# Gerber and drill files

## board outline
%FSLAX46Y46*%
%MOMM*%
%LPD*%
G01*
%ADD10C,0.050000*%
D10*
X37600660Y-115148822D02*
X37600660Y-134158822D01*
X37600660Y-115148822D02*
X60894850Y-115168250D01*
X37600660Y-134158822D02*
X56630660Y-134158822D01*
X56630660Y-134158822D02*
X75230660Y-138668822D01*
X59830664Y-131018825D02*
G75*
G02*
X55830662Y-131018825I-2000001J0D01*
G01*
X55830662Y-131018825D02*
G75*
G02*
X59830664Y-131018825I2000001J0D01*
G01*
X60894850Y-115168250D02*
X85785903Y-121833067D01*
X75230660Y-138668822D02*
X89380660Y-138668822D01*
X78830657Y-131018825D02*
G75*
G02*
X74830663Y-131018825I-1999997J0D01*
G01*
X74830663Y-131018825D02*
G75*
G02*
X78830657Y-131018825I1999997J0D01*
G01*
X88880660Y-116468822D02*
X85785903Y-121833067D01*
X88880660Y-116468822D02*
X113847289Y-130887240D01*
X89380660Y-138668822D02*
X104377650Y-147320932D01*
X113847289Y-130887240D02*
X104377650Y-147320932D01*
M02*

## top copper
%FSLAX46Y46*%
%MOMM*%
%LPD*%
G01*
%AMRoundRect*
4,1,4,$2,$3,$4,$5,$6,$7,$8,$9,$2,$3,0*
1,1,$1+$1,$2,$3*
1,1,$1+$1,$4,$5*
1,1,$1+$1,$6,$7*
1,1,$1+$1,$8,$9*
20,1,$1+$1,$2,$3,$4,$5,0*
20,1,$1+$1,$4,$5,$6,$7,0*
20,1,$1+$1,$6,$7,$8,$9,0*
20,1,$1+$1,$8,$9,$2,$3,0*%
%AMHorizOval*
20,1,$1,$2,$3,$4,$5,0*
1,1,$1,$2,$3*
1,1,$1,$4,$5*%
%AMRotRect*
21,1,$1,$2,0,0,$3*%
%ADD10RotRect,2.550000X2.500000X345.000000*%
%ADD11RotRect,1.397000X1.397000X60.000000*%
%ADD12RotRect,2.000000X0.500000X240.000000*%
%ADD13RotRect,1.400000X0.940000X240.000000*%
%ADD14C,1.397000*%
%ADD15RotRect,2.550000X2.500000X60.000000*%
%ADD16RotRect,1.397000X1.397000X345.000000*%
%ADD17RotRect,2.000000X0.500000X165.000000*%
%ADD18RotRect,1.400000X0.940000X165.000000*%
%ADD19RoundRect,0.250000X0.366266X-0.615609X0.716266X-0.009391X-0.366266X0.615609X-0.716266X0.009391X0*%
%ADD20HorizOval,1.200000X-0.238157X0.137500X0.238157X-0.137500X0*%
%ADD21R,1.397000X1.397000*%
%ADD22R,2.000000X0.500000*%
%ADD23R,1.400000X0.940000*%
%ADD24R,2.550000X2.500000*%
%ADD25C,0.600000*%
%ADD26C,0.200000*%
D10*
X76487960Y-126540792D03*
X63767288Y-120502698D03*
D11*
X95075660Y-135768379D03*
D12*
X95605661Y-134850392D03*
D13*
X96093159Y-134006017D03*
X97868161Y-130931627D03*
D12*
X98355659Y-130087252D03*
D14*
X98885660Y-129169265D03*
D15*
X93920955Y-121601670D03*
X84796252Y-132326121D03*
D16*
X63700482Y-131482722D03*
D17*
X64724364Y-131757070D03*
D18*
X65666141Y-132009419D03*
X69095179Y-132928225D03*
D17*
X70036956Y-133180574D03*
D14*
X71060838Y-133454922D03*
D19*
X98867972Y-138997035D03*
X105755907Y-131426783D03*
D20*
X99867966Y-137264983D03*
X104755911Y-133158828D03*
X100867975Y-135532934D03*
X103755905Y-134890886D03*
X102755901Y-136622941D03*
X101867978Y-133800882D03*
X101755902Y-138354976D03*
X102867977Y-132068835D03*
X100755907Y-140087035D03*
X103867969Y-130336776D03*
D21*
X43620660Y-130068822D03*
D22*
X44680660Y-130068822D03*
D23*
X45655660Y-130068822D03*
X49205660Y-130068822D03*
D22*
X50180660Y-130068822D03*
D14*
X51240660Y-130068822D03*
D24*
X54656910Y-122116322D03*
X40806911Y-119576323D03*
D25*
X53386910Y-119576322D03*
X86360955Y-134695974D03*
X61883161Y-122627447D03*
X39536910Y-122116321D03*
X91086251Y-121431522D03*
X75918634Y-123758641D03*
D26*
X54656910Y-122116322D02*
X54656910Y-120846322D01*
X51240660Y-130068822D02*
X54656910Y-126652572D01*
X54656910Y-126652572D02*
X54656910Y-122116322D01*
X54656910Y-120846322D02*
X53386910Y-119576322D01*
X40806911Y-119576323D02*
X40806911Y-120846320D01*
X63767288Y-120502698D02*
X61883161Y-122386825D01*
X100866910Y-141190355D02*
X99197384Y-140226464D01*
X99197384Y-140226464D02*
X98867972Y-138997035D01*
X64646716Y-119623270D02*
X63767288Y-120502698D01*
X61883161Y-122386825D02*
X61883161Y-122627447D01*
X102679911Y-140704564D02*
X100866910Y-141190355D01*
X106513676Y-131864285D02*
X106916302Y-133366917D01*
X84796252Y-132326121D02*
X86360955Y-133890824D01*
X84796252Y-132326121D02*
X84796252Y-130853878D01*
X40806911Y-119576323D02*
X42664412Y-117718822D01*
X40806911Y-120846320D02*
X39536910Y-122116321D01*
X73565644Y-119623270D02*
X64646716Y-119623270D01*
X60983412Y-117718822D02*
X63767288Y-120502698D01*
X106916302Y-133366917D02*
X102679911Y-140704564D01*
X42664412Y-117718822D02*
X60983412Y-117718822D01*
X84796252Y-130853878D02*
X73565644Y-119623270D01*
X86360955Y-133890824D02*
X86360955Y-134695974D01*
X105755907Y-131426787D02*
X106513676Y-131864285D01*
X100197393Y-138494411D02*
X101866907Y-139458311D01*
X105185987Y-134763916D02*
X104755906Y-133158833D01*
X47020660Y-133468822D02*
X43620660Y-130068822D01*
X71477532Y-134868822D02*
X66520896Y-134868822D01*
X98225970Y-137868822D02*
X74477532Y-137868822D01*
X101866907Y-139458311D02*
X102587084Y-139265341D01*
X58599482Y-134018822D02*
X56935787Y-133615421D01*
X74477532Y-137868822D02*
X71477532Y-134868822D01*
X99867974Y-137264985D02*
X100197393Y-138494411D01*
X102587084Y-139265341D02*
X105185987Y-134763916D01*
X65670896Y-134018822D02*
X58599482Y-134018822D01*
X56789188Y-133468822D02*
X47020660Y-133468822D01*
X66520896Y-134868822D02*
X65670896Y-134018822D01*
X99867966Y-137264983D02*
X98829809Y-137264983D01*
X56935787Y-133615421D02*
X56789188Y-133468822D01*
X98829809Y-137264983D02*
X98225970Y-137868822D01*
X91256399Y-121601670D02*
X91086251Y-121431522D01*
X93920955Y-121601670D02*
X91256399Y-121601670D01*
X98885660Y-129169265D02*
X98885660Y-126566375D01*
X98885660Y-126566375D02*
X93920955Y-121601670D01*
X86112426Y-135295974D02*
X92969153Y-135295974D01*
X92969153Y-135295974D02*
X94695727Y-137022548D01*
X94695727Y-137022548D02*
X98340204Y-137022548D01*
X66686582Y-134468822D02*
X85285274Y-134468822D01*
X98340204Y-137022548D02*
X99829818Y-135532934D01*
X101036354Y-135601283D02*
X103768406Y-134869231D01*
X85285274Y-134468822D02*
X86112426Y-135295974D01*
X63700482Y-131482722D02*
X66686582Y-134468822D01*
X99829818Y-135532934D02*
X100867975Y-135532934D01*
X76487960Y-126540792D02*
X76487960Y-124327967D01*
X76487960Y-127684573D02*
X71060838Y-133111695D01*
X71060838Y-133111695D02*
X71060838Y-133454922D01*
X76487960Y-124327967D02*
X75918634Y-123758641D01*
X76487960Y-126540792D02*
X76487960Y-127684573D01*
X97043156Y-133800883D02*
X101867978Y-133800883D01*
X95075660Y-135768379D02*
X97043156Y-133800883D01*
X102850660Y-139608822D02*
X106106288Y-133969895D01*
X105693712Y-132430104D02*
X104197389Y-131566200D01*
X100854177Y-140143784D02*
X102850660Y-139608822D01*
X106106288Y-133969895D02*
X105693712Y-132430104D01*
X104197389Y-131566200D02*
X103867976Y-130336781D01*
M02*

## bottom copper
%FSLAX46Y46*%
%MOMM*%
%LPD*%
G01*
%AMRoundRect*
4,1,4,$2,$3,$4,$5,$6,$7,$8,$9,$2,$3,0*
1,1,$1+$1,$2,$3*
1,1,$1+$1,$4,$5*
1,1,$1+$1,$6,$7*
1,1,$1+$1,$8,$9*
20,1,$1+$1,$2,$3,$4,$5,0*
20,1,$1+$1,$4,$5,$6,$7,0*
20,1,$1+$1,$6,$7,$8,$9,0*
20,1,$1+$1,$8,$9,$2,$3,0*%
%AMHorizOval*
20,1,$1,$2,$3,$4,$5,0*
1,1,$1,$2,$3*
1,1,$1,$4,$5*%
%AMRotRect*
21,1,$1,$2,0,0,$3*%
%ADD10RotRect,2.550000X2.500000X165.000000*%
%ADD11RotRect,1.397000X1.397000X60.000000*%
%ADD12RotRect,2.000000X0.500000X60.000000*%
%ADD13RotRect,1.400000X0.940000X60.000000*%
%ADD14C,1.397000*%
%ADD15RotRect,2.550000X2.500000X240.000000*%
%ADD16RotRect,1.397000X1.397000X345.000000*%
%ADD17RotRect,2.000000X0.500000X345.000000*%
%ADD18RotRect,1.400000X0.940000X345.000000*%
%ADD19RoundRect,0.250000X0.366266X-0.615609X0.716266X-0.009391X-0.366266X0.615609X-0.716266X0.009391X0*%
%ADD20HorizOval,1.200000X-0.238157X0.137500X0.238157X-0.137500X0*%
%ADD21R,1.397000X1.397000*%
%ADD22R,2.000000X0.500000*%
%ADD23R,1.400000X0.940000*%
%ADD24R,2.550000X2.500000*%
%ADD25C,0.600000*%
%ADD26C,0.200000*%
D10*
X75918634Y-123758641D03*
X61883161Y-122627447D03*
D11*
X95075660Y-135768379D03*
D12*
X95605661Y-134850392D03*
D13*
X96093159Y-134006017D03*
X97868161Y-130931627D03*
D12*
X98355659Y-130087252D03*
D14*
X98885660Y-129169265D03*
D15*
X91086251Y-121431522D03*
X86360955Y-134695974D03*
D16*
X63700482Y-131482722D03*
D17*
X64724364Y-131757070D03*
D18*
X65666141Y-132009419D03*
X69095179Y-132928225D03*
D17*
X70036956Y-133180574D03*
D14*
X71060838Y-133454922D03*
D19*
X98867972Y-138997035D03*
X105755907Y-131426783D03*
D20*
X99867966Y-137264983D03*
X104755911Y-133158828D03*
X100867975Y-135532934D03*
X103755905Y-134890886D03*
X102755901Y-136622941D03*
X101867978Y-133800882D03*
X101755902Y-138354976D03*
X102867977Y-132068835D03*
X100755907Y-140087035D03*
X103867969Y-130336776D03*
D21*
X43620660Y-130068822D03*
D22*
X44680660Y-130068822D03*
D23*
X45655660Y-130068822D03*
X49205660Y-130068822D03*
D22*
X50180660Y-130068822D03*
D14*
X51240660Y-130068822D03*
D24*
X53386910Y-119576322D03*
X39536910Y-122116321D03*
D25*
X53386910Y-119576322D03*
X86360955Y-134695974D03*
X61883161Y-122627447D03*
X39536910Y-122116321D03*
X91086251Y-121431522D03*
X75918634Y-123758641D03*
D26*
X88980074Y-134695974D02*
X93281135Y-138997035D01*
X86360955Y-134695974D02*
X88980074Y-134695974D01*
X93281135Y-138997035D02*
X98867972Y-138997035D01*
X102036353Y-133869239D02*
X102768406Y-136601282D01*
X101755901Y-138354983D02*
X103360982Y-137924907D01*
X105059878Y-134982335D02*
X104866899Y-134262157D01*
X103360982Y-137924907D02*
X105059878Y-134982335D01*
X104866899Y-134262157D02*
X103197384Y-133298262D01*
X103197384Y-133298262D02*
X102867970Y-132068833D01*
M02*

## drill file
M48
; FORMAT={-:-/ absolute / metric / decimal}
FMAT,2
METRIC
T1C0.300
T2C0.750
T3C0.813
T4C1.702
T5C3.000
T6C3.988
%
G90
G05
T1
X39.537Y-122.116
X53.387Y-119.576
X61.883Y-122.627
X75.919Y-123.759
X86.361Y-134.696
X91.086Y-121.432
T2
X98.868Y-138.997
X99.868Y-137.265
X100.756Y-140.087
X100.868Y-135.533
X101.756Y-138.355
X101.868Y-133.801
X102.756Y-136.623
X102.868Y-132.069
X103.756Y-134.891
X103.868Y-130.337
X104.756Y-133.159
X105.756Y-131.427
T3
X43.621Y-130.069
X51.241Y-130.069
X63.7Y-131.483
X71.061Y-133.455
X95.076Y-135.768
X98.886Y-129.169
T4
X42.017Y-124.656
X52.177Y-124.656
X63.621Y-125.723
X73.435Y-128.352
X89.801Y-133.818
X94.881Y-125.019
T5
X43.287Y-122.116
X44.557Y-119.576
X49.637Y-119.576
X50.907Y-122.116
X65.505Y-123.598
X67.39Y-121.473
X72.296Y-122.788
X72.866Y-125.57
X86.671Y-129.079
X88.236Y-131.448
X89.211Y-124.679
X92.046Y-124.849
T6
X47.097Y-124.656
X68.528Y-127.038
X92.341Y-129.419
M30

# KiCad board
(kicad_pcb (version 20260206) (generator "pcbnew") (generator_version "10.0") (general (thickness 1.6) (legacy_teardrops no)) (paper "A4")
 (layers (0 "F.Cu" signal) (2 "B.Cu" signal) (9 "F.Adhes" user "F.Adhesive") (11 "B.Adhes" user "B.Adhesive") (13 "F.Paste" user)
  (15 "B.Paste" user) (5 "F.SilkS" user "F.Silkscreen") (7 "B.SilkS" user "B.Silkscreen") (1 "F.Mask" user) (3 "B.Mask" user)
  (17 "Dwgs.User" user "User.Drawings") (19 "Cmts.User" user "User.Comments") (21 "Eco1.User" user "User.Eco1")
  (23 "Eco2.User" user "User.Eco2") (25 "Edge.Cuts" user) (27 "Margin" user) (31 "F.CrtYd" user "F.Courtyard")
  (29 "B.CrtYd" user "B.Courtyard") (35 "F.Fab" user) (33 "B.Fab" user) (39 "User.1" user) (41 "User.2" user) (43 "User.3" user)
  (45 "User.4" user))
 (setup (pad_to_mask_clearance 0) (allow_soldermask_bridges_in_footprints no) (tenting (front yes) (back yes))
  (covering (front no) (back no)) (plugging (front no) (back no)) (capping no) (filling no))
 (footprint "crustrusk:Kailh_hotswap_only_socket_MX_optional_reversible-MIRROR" (layer "F.Cu") (at 68.52816 127.037572 -15)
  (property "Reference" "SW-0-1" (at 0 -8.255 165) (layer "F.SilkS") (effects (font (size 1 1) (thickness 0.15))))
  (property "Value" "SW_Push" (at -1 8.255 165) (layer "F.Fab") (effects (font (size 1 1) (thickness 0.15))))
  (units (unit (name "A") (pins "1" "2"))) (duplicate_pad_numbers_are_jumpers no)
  (pad "" np_thru_hole circle (at -5.08 0 345) (size 1.7018 1.7018) (drill 1.7018) (layers "*.Cu" "*.Mask"))
  (pad "" np_thru_hole circle (at -3.81 -2.54 165) (size 3 3) (drill 3) (layers "*.Cu" "*.Mask"))
  (pad "" np_thru_hole circle (at -2.54 -5.079998 345) (size 3 3) (drill 3) (layers "*.Cu" "*.Mask"))
  (pad "" np_thru_hole circle (at 0 0 345) (size 3.9878 3.9878) (drill 3.9878) (layers "*.Cu" "*.Mask"))
  (pad "" np_thru_hole circle (at 2.540003 -5.080001 165) (size 3 3) (drill 3) (layers "*.Cu" "*.Mask"))
  (pad "" np_thru_hole circle (at 3.81 -2.54 345) (size 3 3) (drill 3) (layers "*.Cu" "*.Mask"))
  (pad "" np_thru_hole circle (at 5.08 0 345) (size 1.7018 1.7018) (drill 1.7018) (layers "*.Cu" "*.Mask"))
  (pad "1" smd rect (at 6.29 -5.08 165) (size 2.55 2.5) (layers "B.Cu" "B.Mask" "B.Paste") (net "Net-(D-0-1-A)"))
  (pad "1" smd rect (at 7.56 -2.54 345) (size 2.55 2.5) (layers "F.Cu" "F.Mask" "F.Paste") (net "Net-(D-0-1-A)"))
  (pad "2" smd rect (at -7.56 -2.540001 165) (size 2.55 2.5) (layers "B.Cu" "B.Mask" "B.Paste") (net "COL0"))
  (pad "2" smd rect (at -6.289999 -5.079999 345) (size 2.55 2.5) (layers "F.Cu" "F.Mask" "F.Paste") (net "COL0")))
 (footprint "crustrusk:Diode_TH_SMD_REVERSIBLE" (layer "F.Cu") (at 96.98066 132.468822 60)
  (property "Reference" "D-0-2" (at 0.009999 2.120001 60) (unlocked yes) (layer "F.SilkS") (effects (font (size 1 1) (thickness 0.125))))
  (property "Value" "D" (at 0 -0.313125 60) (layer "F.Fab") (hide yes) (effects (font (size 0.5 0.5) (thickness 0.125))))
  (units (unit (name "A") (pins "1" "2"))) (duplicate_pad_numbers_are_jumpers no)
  (pad "1" thru_hole rect (at -3.81 0 60) (size 1.397 1.397) (drill 0.8128) (layers "*.Cu" "*.Mask") (remove_unused_layers no)
   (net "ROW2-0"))
  (pad "1" smd rect (at -2.75 0.000001 240) (size 2 0.5) (layers "F.Cu") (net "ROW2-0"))
  (pad "1" smd rect (at -2.75 0.000001 60) (size 2 0.5) (layers "B.Cu") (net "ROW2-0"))
  (pad "1" smd rect (at -1.775 -0.000001 240) (size 1.4 0.94) (layers "F.Cu" "F.Mask" "F.Paste") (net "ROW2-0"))
  (pad "1" smd rect (at -1.775 -0.000001 60) (size 1.4 0.94) (layers "B.Cu" "B.Mask" "B.Paste") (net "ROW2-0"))
  (pad "2" smd rect (at 1.775 0.000001 240) (size 1.4 0.94) (layers "F.Cu" "F.Mask" "F.Paste") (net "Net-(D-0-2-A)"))
  (pad "2" smd rect (at 1.775 0.000001 60) (size 1.4 0.94) (layers "B.Cu" "B.Mask" "B.Paste") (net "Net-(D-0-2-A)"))
  (pad "2" smd rect (at 2.75 -0.000001 240) (size 2 0.5) (layers "F.Cu") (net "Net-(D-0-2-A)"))
  (pad "2" smd rect (at 2.75 -0.000001 60) (size 2 0.5) (layers "B.Cu") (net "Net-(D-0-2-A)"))
  (pad "2" thru_hole circle (at 3.81 0 60) (size 1.397 1.397) (drill 0.8128) (layers "*.Cu" "*.Mask") (remove_unused_layers no)
   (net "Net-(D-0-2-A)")))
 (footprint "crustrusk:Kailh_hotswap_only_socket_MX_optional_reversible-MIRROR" (layer "F.Cu") (at 92.34066 129.418822 60)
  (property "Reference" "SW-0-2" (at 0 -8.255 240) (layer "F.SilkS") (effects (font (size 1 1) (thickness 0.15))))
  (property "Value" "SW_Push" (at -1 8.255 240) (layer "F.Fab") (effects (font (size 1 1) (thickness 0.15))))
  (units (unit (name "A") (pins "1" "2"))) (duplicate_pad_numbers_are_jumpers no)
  (pad "" np_thru_hole circle (at -5.08 0 60) (size 1.7018 1.7018) (drill 1.7018) (layers "*.Cu" "*.Mask"))
  (pad "" np_thru_hole circle (at -3.81 -2.54 240) (size 3 3) (drill 3) (layers "*.Cu" "*.Mask"))
  (pad "" np_thru_hole circle (at -2.54 -5.079997 60) (size 3 3) (drill 3) (layers "*.Cu" "*.Mask"))
  (pad "" np_thru_hole circle (at 0 0 60) (size 3.9878 3.9878) (drill 3.9878) (layers "*.Cu" "*.Mask"))
  (pad "" np_thru_hole circle (at 2.540002 -5.080001 240) (size 3 3) (drill 3) (layers "*.Cu" "*.Mask"))
  (pad "" np_thru_hole circle (at 3.81 -2.540001 60) (size 3 3) (drill 3) (layers "*.Cu" "*.Mask"))
  (pad "" np_thru_hole circle (at 5.08 0 60) (size 1.7018 1.7018) (drill 1.7018) (layers "*.Cu" "*.Mask"))
  (pad "1" smd rect (at 6.29 -5.08 240) (size 2.55 2.5) (layers "B.Cu" "B.Mask" "B.Paste") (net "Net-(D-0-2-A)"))
  (pad "1" smd rect (at 7.56 -2.54 60) (size 2.55 2.5) (layers "F.Cu" "F.Mask" "F.Paste") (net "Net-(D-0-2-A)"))
  (pad "2" smd rect (at -7.56 -2.54 240) (size 2.55 2.5) (layers "B.Cu" "B.Mask" "B.Paste") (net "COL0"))
  (pad "2" smd rect (at -6.289999 -5.079999 60) (size 2.55 2.5) (layers "F.Cu" "F.Mask" "F.Paste") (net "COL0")))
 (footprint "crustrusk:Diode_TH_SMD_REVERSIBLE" (layer "F.Cu") (at 67.38066 132.468822 -15)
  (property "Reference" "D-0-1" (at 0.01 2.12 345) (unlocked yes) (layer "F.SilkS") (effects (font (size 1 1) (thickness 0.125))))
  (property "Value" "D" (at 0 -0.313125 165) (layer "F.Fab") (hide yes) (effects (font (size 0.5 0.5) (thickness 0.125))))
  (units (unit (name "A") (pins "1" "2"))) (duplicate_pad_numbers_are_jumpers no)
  (pad "1" thru_hole rect (at -3.81 0.000001 345) (size 1.397 1.397) (drill 0.8128) (layers "*.Cu" "*.Mask") (remove_unused_layers no)
   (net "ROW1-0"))
  (pad "1" smd rect (at -2.75 0 165) (size 2 0.5) (layers "F.Cu") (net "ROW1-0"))
  (pad "1" smd rect (at -2.75 0 345) (size 2 0.5) (layers "B.Cu") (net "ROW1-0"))
  (pad "1" smd rect (at -1.775 0.000001 165) (size 1.4 0.94) (layers "F.Cu" "F.Mask" "F.Paste") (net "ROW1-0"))
  (pad "1" smd rect (at -1.775 0.000001 345) (size 1.4 0.94) (layers "B.Cu" "B.Mask" "B.Paste") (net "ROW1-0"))
  (pad "2" smd rect (at 1.775 -0.000001 165) (size 1.4 0.94) (layers "F.Cu" "F.Mask" "F.Paste") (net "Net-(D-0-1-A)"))
  (pad "2" smd rect (at 1.775 -0.000001 345) (size 1.4 0.94) (layers "B.Cu" "B.Mask" "B.Paste") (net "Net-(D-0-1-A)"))
  (pad "2" smd rect (at 2.75 0 165) (size 2 0.5) (layers "F.Cu") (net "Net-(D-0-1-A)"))
  (pad "2" smd rect (at 2.75 0 345) (size 2 0.5) (layers "B.Cu") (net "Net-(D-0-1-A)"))
  (pad "2" thru_hole circle (at 3.81 -0.000001 345) (size 1.397 1.397) (drill 0.8128) (layers "*.Cu" "*.Mask") (remove_unused_layers no)
   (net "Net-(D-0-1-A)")))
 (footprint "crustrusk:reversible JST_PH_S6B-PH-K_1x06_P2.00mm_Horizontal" (layer "F.Cu") (at 98.867972 138.997035 60)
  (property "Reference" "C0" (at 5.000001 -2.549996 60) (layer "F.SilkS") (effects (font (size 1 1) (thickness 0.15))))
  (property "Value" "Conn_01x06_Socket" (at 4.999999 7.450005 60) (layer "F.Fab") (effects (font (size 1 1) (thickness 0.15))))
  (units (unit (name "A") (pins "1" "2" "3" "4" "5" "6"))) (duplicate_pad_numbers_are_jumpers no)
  (pad "1" thru_hole roundrect (at 0 0 60) (size 1.2 1.75) (drill 0.75) (layers "*.Cu" "*.Mask") (remove_unused_layers no)
   (roundrect_rratio 0.208333) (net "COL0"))
  (pad "1" thru_hole roundrect (at 9.999998 2.180001 60) (size 1.2 1.75) (drill 0.75) (layers "*.Cu" "*.Mask") (remove_unused_layers no)
   (roundrect_rratio 0.208333) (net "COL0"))
  (pad "2" thru_hole oval (at 1.999998 -0.000006 60) (size 1.2 1.75) (drill 0.75) (layers "*.Cu" "*.Mask") (remove_unused_layers no)
   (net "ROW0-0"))
  (pad "2" thru_hole oval (at 8.000005 2.180001 60) (size 1.2 1.75) (drill 0.75) (layers "*.Cu" "*.Mask") (remove_unused_layers no)
   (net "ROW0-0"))
  (pad "3" thru_hole oval (at 4.000001 0.000003 60) (size 1.2 1.75) (drill 0.75) (layers "*.Cu" "*.Mask") (remove_unused_layers no)
   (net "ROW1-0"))
  (pad "3" thru_hole oval (at 5.999996 2.18 60) (size 1.2 1.75) (drill 0.75) (layers "*.Cu" "*.Mask") (remove_unused_layers no)
   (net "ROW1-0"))
  (pad "4" thru_hole oval (at 3.99999 2.179998 60) (size 1.2 1.75) (drill 0.75) (layers "*.Cu" "*.Mask") (remove_unused_layers no)
   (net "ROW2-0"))
  (pad "4" thru_hole oval (at 6.000003 0.000005 60) (size 1.2 1.75) (drill 0.75) (layers "*.Cu" "*.Mask") (remove_unused_layers no)
   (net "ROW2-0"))
  (pad "5" thru_hole oval (at 2.000004 2.179991 60) (size 1.2 1.75) (drill 0.75) (layers "*.Cu" "*.Mask") (remove_unused_layers no)
   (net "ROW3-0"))
  (pad "5" thru_hole oval (at 8 0.000006 60) (size 1.2 1.75) (drill 0.75) (layers "*.Cu" "*.Mask") (remove_unused_layers no) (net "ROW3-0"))
  (pad "6" thru_hole oval (at 0 2.18 60) (size 1.2 1.75) (drill 0.75) (layers "*.Cu" "*.Mask") (remove_unused_layers no) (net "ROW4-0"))
  (pad "6" thru_hole oval (at 10.000003 -0.000005 60) (size 1.2 1.75) (drill 0.75) (layers "*.Cu" "*.Mask") (remove_unused_layers no)
   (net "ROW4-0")))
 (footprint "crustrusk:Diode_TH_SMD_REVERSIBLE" (layer "F.Cu") (at 47.43066 130.068822)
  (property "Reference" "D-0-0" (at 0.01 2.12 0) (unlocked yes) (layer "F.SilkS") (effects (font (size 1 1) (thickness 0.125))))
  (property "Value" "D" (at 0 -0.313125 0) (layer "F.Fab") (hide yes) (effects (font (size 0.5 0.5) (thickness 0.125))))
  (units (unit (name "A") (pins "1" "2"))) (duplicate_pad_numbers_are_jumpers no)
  (pad "1" thru_hole rect (at -3.81 0) (size 1.397 1.397) (drill 0.8128) (layers "*.Cu" "*.Mask") (remove_unused_layers no) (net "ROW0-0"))
  (pad "1" smd rect (at -2.75 0 180) (size 2 0.5) (layers "F.Cu") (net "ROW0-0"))
  (pad "1" smd rect (at -2.75 0) (size 2 0.5) (layers "B.Cu") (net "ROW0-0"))
  (pad "1" smd rect (at -1.775 0 180) (size 1.4 0.94) (layers "F.Cu" "F.Mask" "F.Paste") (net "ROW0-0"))
  (pad "1" smd rect (at -1.775 0) (size 1.4 0.94) (layers "B.Cu" "B.Mask" "B.Paste") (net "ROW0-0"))
  (pad "2" smd rect (at 1.775 0 180) (size 1.4 0.94) (layers "F.Cu" "F.Mask" "F.Paste") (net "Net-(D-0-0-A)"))
  (pad "2" smd rect (at 1.775 0) (size 1.4 0.94) (layers "B.Cu" "B.Mask" "B.Paste") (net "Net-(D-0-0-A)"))
  (pad "2" smd rect (at 2.75 0 180) (size 2 0.5) (layers "F.Cu") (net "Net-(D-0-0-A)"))
  (pad "2" smd rect (at 2.75 0) (size 2 0.5) (layers "B.Cu") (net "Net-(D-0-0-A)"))
  (pad "2" thru_hole circle (at 3.81 0) (size 1.397 1.397) (drill 0.8128) (layers "*.Cu" "*.Mask") (remove_unused_layers no)
   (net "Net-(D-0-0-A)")))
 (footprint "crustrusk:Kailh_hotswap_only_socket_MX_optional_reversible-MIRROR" (layer "F.Cu") (at 47.09691 124.656322)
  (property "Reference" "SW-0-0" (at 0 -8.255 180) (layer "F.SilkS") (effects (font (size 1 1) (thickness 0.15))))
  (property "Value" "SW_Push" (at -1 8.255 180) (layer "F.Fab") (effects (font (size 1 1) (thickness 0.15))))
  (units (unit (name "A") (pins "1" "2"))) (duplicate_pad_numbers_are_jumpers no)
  (pad "" np_thru_hole circle (at -5.08 0) (size 1.7018 1.7018) (drill 1.7018) (layers "*.Cu" "*.Mask"))
  (pad "" np_thru_hole circle (at -3.81 -2.54 180) (size 3 3) (drill 3) (layers "*.Cu" "*.Mask"))
  (pad "" np_thru_hole circle (at -2.54 -5.079998) (size 3 3) (drill 3) (layers "*.Cu" "*.Mask"))
  (pad "" np_thru_hole circle (at 0 0) (size 3.9878 3.9878) (drill 3.9878) (layers "*.Cu" "*.Mask"))
  (pad "" np_thru_hole circle (at 2.540002 -5.080001 180) (size 3 3) (drill 3) (layers "*.Cu" "*.Mask"))
  (pad "" np_thru_hole circle (at 3.81 -2.54) (size 3 3) (drill 3) (layers "*.Cu" "*.Mask"))
  (pad "" np_thru_hole circle (at 5.08 0) (size 1.7018 1.7018) (drill 1.7018) (layers "*.Cu" "*.Mask"))
  (pad "1" smd rect (at 6.29 -5.08 180) (size 2.55 2.5) (layers "B.Cu" "B.Mask" "B.Paste") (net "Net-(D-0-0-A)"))
  (pad "1" smd rect (at 7.56 -2.54) (size 2.55 2.5) (layers "F.Cu" "F.Mask" "F.Paste") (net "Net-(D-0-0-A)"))
  (pad "2" smd rect (at -7.56 -2.540001 180) (size 2.55 2.5) (layers "B.Cu" "B.Mask" "B.Paste") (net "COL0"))
  (pad "2" smd rect (at -6.289999 -5.079999) (size 2.55 2.5) (layers "F.Cu" "F.Mask" "F.Paste") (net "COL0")))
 (gr_line (start 37.60066 115.148822) (end 37.60066 134.158822) (stroke (width 0.05) (type default)) (layer "Edge.Cuts"))
 (gr_line (start 37.60066 115.148822) (end 60.89485 115.16825) (stroke (width 0.05) (type default)) (layer "Edge.Cuts"))
 (gr_line (start 37.60066 134.158822) (end 56.63066 134.158822) (stroke (width 0.05) (type default)) (layer "Edge.Cuts"))
 (gr_line (start 56.63066 134.158822) (end 75.23066 138.668822) (stroke (width 0.05) (type default)) (layer "Edge.Cuts"))
 (gr_circle (center 57.830663 131.018825) (end 55.830662 131.018825) (stroke (width 0.05) (type default)) (fill no) (layer "Edge.Cuts"))
 (gr_line (start 60.89485 115.16825) (end 85.785903 121.833067) (stroke (width 0.05) (type default)) (layer "Edge.Cuts"))
 (gr_line (start 75.23066 138.668822) (end 89.38066 138.668822) (stroke (width 0.05) (type default)) (layer "Edge.Cuts"))
 (gr_circle (center 76.83066 131.018825) (end 74.830663 131.018825) (stroke (width 0.05) (type default)) (fill no) (layer "Edge.Cuts"))
 (gr_line (start 88.88066 116.468822) (end 85.785903 121.833067) (stroke (width 0.05) (type default)) (layer "Edge.Cuts"))
 (gr_line (start 88.88066 116.468822) (end 113.847289 130.88724) (stroke (width 0.05) (type default)) (layer "Edge.Cuts"))
 (gr_line (start 89.38066 138.668822) (end 104.37765 147.320932) (stroke (width 0.05) (type default)) (layer "Edge.Cuts"))
 (gr_line (start 113.847289 130.88724) (end 104.37765 147.320932) (stroke (width 0.05) (type default)) (layer "Edge.Cuts"))
 (segment (start 54.65691 122.116322) (end 54.65691 120.846322) (width 0.2) (layer "F.Cu") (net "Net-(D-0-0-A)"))
 (segment (start 51.24066 130.068822) (end 54.65691 126.652572) (width 0.2) (layer "F.Cu") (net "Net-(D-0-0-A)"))
 (segment (start 54.65691 126.652572) (end 54.65691 122.116322) (width 0.2) (layer "F.Cu") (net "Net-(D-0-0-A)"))
 (segment (start 54.65691 120.846322) (end 53.38691 119.576322) (width 0.2) (layer "F.Cu") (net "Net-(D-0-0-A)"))
 (via (at 53.38691 119.576322) (size 0.6) (drill 0.3) (layers "F.Cu" "B.Cu") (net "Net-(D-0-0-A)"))
 (segment (start 40.806911 119.576323) (end 40.806911 120.84632) (width 0.2) (layer "F.Cu") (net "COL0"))
 (segment (start 63.767288 120.502698) (end 61.883161 122.386825) (width 0.2) (layer "F.Cu") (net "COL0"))
 (segment (start 100.86691 141.190355) (end 99.197384 140.226464) (width 0.2) (layer "F.Cu") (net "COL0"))
 (segment (start 99.197384 140.226464) (end 98.867972 138.997035) (width 0.2) (layer "F.Cu") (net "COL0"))
 (segment (start 64.646716 119.62327) (end 63.767288 120.502698) (width 0.2) (layer "F.Cu") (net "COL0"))
 (segment (start 61.883161 122.386825) (end 61.883161 122.627447) (width 0.2) (layer "F.Cu") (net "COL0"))
 (segment (start 102.679911 140.704564) (end 100.86691 141.190355) (width 0.2) (layer "F.Cu") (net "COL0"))
 (segment (start 106.513676 131.864285) (end 106.916302 133.366917) (width 0.2) (layer "F.Cu") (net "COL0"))
 (segment (start 84.796252 132.326121) (end 86.360955 133.890824) (width 0.2) (layer "F.Cu") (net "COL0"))
 (segment (start 84.796252 132.326121) (end 84.796252 130.853878) (width 0.2) (layer "F.Cu") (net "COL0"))
 (segment (start 40.806911 119.576323) (end 42.664412 117.718822) (width 0.2) (layer "F.Cu") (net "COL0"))
 (segment (start 40.806911 120.84632) (end 39.53691 122.116321) (width 0.2) (layer "F.Cu") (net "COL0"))
 (segment (start 73.565644 119.62327) (end 64.646716 119.62327) (width 0.2) (layer "F.Cu") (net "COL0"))
 (segment (start 60.983412 117.718822) (end 63.767288 120.502698) (width 0.2) (layer "F.Cu") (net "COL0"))
 (segment (start 106.916302 133.366917) (end 102.679911 140.704564) (width 0.2) (layer "F.Cu") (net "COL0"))
 (segment (start 42.664412 117.718822) (end 60.983412 117.718822) (width 0.2) (layer "F.Cu") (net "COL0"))
 (segment (start 84.796252 130.853878) (end 73.565644 119.62327) (width 0.2) (layer "F.Cu") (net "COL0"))
 (segment (start 86.360955 133.890824) (end 86.360955 134.695974) (width 0.2) (layer "F.Cu") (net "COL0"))
 (segment (start 105.755907 131.426787) (end 106.513676 131.864285) (width 0.2) (layer "F.Cu") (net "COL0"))
 (via (at 86.360955 134.695974) (size 0.6) (drill 0.3) (layers "F.Cu" "B.Cu") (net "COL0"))
 (via (at 61.883161 122.627447) (size 0.6) (drill 0.3) (layers "F.Cu" "B.Cu") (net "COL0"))
 (via (at 39.53691 122.116321) (size 0.6) (drill 0.3) (layers "F.Cu" "B.Cu") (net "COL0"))
 (segment (start 88.980074 134.695974) (end 93.281135 138.997035) (width 0.2) (layer "B.Cu") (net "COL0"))
 (segment (start 86.360955 134.695974) (end 88.980074 134.695974) (width 0.2) (layer "B.Cu") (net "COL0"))
 (segment (start 93.281135 138.997035) (end 98.867972 138.997035) (width 0.2) (layer "B.Cu") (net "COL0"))
 (segment (start 100.197393 138.494411) (end 101.866907 139.458311) (width 0.2) (layer "F.Cu") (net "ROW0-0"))
 (segment (start 105.185987 134.763916) (end 104.755906 133.158833) (width 0.2) (layer "F.Cu") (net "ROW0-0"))
 (segment (start 47.02066 133.468822) (end 43.62066 130.068822) (width 0.2) (layer "F.Cu") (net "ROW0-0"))
 (segment (start 71.477532 134.868822) (end 66.520896 134.868822) (width 0.2) (layer "F.Cu") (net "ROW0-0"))
 (segment (start 98.22597 137.868822) (end 74.477532 137.868822) (width 0.2) (layer "F.Cu") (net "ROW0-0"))
 (segment (start 101.866907 139.458311) (end 102.587084 139.265341) (width 0.2) (layer "F.Cu") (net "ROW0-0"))
 (segment (start 58.599482 134.018822) (end 56.935787 133.615421) (width 0.2) (layer "F.Cu") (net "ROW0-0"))
 (segment (start 74.477532 137.868822) (end 71.477532 134.868822) (width 0.2) (layer "F.Cu") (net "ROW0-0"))
 (segment (start 99.867974 137.264985) (end 100.197393 138.494411) (width 0.2) (layer "F.Cu") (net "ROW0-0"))
 (segment (start 102.587084 139.265341) (end 105.185987 134.763916) (width 0.2) (layer "F.Cu") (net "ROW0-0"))
 (segment (start 65.670896 134.018822) (end 58.599482 134.018822) (width 0.2) (layer "F.Cu") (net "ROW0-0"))
 (segment (start 56.789188 133.468822) (end 47.02066 133.468822) (width 0.2) (layer "F.Cu") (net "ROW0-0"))
 (segment (start 66.520896 134.868822) (end 65.670896 134.018822) (width 0.2) (layer "F.Cu") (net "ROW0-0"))
 (segment (start 99.867966 137.264983) (end 98.829809 137.264983) (width 0.2) (layer "F.Cu") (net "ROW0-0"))
 (segment (start 56.935787 133.615421) (end 56.789188 133.468822) (width 0.2) (layer "F.Cu") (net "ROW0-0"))
 (segment (start 98.829809 137.264983) (end 98.22597 137.868822) (width 0.2) (layer "F.Cu") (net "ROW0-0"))
 (segment (start 91.256399 121.60167) (end 91.086251 121.431522) (width 0.2) (layer "F.Cu") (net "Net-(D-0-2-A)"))
 (segment (start 93.920955 121.60167) (end 91.256399 121.60167) (width 0.2) (layer "F.Cu") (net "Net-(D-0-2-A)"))
 (segment (start 98.88566 129.169265) (end 98.88566 126.566375) (width 0.2) (layer "F.Cu") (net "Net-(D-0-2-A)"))
 (segment (start 98.88566 126.566375) (end 93.920955 121.60167) (width 0.2) (layer "F.Cu") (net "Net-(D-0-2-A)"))
 (via (at 91.086251 121.431522) (size 0.6) (drill 0.3) (layers "F.Cu" "B.Cu") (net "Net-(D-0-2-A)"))
 (segment (start 86.112426 135.295974) (end 92.969153 135.295974) (width 0.2) (layer "F.Cu") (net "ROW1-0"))
 (segment (start 92.969153 135.295974) (end 94.695727 137.022548) (width 0.2) (layer "F.Cu") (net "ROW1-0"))
 (segment (start 94.695727 137.022548) (end 98.340204 137.022548) (width 0.2) (layer "F.Cu") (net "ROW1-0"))
 (segment (start 66.686582 134.468822) (end 85.285274 134.468822) (width 0.2) (layer "F.Cu") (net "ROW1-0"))
 (segment (start 98.340204 137.022548) (end 99.829818 135.532934) (width 0.2) (layer "F.Cu") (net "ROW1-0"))
 (segment (start 101.036354 135.601283) (end 103.768406 134.869231) (width 0.2) (layer "F.Cu") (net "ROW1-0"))
 (segment (start 85.285274 134.468822) (end 86.112426 135.295974) (width 0.2) (layer "F.Cu") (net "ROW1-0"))
 (segment (start 63.700482 131.482722) (end 66.686582 134.468822) (width 0.2) (layer "F.Cu") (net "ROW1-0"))
 (segment (start 99.829818 135.532934) (end 100.867975 135.532934) (width 0.2) (layer "F.Cu") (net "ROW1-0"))
 (segment (start 76.48796 126.540792) (end 76.48796 124.327967) (width 0.2) (layer "F.Cu") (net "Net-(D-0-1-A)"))
 (segment (start 76.48796 127.684573) (end 71.060838 133.111695) (width 0.2) (layer "F.Cu") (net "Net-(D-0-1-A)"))
 (segment (start 71.060838 133.111695) (end 71.060838 133.454922) (width 0.2) (layer "F.Cu") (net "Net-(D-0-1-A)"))
 (segment (start 76.48796 124.327967) (end 75.918634 123.758641) (width 0.2) (layer "F.Cu") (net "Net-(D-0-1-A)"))
 (segment (start 76.48796 126.540792) (end 76.48796 127.684573) (width 0.2) (layer "F.Cu") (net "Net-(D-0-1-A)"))
 (via (at 75.918634 123.758641) (size 0.6) (drill 0.3) (layers "F.Cu" "B.Cu") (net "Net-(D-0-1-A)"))
 (segment (start 97.043156 133.800883) (end 101.867978 133.800883) (width 0.2) (layer "F.Cu") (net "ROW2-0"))
 (segment (start 95.07566 135.768379) (end 97.043156 133.800883) (width 0.2) (layer "F.Cu") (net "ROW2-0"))
 (segment (start 102.036353 133.869239) (end 102.768406 136.601282) (width 0.2) (layer "B.Cu") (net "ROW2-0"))
 (segment (start 101.755901 138.354983) (end 103.360982 137.924907) (width 0.2) (layer "B.Cu") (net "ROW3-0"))
 (segment (start 105.059878 134.982335) (end 104.866899 134.262157) (width 0.2) (layer "B.Cu") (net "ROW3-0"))
 (segment (start 103.360982 137.924907) (end 105.059878 134.982335) (width 0.2) (layer "B.Cu") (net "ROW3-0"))
 (segment (start 104.866899 134.262157) (end 103.197384 133.298262) (width 0.2) (layer "B.Cu") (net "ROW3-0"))
 (segment (start 103.197384 133.298262) (end 102.86797 132.068833) (width 0.2) (layer "B.Cu") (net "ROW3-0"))
 (segment (start 102.85066 139.608822) (end 106.106288 133.969895) (width 0.2) (layer "F.Cu") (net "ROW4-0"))
 (segment (start 105.693712 132.430104) (end 104.197389 131.5662) (width 0.2) (layer "F.Cu") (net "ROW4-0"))
 (segment (start 100.854177 140.143784) (end 102.85066 139.608822) (width 0.2) (layer "F.Cu") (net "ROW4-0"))
 (segment (start 106.106288 133.969895) (end 105.693712 132.430104) (width 0.2) (layer "F.Cu") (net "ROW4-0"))
 (segment (start 104.197389 131.5662) (end 103.867976 130.336781) (width 0.2) (layer "F.Cu") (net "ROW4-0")))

